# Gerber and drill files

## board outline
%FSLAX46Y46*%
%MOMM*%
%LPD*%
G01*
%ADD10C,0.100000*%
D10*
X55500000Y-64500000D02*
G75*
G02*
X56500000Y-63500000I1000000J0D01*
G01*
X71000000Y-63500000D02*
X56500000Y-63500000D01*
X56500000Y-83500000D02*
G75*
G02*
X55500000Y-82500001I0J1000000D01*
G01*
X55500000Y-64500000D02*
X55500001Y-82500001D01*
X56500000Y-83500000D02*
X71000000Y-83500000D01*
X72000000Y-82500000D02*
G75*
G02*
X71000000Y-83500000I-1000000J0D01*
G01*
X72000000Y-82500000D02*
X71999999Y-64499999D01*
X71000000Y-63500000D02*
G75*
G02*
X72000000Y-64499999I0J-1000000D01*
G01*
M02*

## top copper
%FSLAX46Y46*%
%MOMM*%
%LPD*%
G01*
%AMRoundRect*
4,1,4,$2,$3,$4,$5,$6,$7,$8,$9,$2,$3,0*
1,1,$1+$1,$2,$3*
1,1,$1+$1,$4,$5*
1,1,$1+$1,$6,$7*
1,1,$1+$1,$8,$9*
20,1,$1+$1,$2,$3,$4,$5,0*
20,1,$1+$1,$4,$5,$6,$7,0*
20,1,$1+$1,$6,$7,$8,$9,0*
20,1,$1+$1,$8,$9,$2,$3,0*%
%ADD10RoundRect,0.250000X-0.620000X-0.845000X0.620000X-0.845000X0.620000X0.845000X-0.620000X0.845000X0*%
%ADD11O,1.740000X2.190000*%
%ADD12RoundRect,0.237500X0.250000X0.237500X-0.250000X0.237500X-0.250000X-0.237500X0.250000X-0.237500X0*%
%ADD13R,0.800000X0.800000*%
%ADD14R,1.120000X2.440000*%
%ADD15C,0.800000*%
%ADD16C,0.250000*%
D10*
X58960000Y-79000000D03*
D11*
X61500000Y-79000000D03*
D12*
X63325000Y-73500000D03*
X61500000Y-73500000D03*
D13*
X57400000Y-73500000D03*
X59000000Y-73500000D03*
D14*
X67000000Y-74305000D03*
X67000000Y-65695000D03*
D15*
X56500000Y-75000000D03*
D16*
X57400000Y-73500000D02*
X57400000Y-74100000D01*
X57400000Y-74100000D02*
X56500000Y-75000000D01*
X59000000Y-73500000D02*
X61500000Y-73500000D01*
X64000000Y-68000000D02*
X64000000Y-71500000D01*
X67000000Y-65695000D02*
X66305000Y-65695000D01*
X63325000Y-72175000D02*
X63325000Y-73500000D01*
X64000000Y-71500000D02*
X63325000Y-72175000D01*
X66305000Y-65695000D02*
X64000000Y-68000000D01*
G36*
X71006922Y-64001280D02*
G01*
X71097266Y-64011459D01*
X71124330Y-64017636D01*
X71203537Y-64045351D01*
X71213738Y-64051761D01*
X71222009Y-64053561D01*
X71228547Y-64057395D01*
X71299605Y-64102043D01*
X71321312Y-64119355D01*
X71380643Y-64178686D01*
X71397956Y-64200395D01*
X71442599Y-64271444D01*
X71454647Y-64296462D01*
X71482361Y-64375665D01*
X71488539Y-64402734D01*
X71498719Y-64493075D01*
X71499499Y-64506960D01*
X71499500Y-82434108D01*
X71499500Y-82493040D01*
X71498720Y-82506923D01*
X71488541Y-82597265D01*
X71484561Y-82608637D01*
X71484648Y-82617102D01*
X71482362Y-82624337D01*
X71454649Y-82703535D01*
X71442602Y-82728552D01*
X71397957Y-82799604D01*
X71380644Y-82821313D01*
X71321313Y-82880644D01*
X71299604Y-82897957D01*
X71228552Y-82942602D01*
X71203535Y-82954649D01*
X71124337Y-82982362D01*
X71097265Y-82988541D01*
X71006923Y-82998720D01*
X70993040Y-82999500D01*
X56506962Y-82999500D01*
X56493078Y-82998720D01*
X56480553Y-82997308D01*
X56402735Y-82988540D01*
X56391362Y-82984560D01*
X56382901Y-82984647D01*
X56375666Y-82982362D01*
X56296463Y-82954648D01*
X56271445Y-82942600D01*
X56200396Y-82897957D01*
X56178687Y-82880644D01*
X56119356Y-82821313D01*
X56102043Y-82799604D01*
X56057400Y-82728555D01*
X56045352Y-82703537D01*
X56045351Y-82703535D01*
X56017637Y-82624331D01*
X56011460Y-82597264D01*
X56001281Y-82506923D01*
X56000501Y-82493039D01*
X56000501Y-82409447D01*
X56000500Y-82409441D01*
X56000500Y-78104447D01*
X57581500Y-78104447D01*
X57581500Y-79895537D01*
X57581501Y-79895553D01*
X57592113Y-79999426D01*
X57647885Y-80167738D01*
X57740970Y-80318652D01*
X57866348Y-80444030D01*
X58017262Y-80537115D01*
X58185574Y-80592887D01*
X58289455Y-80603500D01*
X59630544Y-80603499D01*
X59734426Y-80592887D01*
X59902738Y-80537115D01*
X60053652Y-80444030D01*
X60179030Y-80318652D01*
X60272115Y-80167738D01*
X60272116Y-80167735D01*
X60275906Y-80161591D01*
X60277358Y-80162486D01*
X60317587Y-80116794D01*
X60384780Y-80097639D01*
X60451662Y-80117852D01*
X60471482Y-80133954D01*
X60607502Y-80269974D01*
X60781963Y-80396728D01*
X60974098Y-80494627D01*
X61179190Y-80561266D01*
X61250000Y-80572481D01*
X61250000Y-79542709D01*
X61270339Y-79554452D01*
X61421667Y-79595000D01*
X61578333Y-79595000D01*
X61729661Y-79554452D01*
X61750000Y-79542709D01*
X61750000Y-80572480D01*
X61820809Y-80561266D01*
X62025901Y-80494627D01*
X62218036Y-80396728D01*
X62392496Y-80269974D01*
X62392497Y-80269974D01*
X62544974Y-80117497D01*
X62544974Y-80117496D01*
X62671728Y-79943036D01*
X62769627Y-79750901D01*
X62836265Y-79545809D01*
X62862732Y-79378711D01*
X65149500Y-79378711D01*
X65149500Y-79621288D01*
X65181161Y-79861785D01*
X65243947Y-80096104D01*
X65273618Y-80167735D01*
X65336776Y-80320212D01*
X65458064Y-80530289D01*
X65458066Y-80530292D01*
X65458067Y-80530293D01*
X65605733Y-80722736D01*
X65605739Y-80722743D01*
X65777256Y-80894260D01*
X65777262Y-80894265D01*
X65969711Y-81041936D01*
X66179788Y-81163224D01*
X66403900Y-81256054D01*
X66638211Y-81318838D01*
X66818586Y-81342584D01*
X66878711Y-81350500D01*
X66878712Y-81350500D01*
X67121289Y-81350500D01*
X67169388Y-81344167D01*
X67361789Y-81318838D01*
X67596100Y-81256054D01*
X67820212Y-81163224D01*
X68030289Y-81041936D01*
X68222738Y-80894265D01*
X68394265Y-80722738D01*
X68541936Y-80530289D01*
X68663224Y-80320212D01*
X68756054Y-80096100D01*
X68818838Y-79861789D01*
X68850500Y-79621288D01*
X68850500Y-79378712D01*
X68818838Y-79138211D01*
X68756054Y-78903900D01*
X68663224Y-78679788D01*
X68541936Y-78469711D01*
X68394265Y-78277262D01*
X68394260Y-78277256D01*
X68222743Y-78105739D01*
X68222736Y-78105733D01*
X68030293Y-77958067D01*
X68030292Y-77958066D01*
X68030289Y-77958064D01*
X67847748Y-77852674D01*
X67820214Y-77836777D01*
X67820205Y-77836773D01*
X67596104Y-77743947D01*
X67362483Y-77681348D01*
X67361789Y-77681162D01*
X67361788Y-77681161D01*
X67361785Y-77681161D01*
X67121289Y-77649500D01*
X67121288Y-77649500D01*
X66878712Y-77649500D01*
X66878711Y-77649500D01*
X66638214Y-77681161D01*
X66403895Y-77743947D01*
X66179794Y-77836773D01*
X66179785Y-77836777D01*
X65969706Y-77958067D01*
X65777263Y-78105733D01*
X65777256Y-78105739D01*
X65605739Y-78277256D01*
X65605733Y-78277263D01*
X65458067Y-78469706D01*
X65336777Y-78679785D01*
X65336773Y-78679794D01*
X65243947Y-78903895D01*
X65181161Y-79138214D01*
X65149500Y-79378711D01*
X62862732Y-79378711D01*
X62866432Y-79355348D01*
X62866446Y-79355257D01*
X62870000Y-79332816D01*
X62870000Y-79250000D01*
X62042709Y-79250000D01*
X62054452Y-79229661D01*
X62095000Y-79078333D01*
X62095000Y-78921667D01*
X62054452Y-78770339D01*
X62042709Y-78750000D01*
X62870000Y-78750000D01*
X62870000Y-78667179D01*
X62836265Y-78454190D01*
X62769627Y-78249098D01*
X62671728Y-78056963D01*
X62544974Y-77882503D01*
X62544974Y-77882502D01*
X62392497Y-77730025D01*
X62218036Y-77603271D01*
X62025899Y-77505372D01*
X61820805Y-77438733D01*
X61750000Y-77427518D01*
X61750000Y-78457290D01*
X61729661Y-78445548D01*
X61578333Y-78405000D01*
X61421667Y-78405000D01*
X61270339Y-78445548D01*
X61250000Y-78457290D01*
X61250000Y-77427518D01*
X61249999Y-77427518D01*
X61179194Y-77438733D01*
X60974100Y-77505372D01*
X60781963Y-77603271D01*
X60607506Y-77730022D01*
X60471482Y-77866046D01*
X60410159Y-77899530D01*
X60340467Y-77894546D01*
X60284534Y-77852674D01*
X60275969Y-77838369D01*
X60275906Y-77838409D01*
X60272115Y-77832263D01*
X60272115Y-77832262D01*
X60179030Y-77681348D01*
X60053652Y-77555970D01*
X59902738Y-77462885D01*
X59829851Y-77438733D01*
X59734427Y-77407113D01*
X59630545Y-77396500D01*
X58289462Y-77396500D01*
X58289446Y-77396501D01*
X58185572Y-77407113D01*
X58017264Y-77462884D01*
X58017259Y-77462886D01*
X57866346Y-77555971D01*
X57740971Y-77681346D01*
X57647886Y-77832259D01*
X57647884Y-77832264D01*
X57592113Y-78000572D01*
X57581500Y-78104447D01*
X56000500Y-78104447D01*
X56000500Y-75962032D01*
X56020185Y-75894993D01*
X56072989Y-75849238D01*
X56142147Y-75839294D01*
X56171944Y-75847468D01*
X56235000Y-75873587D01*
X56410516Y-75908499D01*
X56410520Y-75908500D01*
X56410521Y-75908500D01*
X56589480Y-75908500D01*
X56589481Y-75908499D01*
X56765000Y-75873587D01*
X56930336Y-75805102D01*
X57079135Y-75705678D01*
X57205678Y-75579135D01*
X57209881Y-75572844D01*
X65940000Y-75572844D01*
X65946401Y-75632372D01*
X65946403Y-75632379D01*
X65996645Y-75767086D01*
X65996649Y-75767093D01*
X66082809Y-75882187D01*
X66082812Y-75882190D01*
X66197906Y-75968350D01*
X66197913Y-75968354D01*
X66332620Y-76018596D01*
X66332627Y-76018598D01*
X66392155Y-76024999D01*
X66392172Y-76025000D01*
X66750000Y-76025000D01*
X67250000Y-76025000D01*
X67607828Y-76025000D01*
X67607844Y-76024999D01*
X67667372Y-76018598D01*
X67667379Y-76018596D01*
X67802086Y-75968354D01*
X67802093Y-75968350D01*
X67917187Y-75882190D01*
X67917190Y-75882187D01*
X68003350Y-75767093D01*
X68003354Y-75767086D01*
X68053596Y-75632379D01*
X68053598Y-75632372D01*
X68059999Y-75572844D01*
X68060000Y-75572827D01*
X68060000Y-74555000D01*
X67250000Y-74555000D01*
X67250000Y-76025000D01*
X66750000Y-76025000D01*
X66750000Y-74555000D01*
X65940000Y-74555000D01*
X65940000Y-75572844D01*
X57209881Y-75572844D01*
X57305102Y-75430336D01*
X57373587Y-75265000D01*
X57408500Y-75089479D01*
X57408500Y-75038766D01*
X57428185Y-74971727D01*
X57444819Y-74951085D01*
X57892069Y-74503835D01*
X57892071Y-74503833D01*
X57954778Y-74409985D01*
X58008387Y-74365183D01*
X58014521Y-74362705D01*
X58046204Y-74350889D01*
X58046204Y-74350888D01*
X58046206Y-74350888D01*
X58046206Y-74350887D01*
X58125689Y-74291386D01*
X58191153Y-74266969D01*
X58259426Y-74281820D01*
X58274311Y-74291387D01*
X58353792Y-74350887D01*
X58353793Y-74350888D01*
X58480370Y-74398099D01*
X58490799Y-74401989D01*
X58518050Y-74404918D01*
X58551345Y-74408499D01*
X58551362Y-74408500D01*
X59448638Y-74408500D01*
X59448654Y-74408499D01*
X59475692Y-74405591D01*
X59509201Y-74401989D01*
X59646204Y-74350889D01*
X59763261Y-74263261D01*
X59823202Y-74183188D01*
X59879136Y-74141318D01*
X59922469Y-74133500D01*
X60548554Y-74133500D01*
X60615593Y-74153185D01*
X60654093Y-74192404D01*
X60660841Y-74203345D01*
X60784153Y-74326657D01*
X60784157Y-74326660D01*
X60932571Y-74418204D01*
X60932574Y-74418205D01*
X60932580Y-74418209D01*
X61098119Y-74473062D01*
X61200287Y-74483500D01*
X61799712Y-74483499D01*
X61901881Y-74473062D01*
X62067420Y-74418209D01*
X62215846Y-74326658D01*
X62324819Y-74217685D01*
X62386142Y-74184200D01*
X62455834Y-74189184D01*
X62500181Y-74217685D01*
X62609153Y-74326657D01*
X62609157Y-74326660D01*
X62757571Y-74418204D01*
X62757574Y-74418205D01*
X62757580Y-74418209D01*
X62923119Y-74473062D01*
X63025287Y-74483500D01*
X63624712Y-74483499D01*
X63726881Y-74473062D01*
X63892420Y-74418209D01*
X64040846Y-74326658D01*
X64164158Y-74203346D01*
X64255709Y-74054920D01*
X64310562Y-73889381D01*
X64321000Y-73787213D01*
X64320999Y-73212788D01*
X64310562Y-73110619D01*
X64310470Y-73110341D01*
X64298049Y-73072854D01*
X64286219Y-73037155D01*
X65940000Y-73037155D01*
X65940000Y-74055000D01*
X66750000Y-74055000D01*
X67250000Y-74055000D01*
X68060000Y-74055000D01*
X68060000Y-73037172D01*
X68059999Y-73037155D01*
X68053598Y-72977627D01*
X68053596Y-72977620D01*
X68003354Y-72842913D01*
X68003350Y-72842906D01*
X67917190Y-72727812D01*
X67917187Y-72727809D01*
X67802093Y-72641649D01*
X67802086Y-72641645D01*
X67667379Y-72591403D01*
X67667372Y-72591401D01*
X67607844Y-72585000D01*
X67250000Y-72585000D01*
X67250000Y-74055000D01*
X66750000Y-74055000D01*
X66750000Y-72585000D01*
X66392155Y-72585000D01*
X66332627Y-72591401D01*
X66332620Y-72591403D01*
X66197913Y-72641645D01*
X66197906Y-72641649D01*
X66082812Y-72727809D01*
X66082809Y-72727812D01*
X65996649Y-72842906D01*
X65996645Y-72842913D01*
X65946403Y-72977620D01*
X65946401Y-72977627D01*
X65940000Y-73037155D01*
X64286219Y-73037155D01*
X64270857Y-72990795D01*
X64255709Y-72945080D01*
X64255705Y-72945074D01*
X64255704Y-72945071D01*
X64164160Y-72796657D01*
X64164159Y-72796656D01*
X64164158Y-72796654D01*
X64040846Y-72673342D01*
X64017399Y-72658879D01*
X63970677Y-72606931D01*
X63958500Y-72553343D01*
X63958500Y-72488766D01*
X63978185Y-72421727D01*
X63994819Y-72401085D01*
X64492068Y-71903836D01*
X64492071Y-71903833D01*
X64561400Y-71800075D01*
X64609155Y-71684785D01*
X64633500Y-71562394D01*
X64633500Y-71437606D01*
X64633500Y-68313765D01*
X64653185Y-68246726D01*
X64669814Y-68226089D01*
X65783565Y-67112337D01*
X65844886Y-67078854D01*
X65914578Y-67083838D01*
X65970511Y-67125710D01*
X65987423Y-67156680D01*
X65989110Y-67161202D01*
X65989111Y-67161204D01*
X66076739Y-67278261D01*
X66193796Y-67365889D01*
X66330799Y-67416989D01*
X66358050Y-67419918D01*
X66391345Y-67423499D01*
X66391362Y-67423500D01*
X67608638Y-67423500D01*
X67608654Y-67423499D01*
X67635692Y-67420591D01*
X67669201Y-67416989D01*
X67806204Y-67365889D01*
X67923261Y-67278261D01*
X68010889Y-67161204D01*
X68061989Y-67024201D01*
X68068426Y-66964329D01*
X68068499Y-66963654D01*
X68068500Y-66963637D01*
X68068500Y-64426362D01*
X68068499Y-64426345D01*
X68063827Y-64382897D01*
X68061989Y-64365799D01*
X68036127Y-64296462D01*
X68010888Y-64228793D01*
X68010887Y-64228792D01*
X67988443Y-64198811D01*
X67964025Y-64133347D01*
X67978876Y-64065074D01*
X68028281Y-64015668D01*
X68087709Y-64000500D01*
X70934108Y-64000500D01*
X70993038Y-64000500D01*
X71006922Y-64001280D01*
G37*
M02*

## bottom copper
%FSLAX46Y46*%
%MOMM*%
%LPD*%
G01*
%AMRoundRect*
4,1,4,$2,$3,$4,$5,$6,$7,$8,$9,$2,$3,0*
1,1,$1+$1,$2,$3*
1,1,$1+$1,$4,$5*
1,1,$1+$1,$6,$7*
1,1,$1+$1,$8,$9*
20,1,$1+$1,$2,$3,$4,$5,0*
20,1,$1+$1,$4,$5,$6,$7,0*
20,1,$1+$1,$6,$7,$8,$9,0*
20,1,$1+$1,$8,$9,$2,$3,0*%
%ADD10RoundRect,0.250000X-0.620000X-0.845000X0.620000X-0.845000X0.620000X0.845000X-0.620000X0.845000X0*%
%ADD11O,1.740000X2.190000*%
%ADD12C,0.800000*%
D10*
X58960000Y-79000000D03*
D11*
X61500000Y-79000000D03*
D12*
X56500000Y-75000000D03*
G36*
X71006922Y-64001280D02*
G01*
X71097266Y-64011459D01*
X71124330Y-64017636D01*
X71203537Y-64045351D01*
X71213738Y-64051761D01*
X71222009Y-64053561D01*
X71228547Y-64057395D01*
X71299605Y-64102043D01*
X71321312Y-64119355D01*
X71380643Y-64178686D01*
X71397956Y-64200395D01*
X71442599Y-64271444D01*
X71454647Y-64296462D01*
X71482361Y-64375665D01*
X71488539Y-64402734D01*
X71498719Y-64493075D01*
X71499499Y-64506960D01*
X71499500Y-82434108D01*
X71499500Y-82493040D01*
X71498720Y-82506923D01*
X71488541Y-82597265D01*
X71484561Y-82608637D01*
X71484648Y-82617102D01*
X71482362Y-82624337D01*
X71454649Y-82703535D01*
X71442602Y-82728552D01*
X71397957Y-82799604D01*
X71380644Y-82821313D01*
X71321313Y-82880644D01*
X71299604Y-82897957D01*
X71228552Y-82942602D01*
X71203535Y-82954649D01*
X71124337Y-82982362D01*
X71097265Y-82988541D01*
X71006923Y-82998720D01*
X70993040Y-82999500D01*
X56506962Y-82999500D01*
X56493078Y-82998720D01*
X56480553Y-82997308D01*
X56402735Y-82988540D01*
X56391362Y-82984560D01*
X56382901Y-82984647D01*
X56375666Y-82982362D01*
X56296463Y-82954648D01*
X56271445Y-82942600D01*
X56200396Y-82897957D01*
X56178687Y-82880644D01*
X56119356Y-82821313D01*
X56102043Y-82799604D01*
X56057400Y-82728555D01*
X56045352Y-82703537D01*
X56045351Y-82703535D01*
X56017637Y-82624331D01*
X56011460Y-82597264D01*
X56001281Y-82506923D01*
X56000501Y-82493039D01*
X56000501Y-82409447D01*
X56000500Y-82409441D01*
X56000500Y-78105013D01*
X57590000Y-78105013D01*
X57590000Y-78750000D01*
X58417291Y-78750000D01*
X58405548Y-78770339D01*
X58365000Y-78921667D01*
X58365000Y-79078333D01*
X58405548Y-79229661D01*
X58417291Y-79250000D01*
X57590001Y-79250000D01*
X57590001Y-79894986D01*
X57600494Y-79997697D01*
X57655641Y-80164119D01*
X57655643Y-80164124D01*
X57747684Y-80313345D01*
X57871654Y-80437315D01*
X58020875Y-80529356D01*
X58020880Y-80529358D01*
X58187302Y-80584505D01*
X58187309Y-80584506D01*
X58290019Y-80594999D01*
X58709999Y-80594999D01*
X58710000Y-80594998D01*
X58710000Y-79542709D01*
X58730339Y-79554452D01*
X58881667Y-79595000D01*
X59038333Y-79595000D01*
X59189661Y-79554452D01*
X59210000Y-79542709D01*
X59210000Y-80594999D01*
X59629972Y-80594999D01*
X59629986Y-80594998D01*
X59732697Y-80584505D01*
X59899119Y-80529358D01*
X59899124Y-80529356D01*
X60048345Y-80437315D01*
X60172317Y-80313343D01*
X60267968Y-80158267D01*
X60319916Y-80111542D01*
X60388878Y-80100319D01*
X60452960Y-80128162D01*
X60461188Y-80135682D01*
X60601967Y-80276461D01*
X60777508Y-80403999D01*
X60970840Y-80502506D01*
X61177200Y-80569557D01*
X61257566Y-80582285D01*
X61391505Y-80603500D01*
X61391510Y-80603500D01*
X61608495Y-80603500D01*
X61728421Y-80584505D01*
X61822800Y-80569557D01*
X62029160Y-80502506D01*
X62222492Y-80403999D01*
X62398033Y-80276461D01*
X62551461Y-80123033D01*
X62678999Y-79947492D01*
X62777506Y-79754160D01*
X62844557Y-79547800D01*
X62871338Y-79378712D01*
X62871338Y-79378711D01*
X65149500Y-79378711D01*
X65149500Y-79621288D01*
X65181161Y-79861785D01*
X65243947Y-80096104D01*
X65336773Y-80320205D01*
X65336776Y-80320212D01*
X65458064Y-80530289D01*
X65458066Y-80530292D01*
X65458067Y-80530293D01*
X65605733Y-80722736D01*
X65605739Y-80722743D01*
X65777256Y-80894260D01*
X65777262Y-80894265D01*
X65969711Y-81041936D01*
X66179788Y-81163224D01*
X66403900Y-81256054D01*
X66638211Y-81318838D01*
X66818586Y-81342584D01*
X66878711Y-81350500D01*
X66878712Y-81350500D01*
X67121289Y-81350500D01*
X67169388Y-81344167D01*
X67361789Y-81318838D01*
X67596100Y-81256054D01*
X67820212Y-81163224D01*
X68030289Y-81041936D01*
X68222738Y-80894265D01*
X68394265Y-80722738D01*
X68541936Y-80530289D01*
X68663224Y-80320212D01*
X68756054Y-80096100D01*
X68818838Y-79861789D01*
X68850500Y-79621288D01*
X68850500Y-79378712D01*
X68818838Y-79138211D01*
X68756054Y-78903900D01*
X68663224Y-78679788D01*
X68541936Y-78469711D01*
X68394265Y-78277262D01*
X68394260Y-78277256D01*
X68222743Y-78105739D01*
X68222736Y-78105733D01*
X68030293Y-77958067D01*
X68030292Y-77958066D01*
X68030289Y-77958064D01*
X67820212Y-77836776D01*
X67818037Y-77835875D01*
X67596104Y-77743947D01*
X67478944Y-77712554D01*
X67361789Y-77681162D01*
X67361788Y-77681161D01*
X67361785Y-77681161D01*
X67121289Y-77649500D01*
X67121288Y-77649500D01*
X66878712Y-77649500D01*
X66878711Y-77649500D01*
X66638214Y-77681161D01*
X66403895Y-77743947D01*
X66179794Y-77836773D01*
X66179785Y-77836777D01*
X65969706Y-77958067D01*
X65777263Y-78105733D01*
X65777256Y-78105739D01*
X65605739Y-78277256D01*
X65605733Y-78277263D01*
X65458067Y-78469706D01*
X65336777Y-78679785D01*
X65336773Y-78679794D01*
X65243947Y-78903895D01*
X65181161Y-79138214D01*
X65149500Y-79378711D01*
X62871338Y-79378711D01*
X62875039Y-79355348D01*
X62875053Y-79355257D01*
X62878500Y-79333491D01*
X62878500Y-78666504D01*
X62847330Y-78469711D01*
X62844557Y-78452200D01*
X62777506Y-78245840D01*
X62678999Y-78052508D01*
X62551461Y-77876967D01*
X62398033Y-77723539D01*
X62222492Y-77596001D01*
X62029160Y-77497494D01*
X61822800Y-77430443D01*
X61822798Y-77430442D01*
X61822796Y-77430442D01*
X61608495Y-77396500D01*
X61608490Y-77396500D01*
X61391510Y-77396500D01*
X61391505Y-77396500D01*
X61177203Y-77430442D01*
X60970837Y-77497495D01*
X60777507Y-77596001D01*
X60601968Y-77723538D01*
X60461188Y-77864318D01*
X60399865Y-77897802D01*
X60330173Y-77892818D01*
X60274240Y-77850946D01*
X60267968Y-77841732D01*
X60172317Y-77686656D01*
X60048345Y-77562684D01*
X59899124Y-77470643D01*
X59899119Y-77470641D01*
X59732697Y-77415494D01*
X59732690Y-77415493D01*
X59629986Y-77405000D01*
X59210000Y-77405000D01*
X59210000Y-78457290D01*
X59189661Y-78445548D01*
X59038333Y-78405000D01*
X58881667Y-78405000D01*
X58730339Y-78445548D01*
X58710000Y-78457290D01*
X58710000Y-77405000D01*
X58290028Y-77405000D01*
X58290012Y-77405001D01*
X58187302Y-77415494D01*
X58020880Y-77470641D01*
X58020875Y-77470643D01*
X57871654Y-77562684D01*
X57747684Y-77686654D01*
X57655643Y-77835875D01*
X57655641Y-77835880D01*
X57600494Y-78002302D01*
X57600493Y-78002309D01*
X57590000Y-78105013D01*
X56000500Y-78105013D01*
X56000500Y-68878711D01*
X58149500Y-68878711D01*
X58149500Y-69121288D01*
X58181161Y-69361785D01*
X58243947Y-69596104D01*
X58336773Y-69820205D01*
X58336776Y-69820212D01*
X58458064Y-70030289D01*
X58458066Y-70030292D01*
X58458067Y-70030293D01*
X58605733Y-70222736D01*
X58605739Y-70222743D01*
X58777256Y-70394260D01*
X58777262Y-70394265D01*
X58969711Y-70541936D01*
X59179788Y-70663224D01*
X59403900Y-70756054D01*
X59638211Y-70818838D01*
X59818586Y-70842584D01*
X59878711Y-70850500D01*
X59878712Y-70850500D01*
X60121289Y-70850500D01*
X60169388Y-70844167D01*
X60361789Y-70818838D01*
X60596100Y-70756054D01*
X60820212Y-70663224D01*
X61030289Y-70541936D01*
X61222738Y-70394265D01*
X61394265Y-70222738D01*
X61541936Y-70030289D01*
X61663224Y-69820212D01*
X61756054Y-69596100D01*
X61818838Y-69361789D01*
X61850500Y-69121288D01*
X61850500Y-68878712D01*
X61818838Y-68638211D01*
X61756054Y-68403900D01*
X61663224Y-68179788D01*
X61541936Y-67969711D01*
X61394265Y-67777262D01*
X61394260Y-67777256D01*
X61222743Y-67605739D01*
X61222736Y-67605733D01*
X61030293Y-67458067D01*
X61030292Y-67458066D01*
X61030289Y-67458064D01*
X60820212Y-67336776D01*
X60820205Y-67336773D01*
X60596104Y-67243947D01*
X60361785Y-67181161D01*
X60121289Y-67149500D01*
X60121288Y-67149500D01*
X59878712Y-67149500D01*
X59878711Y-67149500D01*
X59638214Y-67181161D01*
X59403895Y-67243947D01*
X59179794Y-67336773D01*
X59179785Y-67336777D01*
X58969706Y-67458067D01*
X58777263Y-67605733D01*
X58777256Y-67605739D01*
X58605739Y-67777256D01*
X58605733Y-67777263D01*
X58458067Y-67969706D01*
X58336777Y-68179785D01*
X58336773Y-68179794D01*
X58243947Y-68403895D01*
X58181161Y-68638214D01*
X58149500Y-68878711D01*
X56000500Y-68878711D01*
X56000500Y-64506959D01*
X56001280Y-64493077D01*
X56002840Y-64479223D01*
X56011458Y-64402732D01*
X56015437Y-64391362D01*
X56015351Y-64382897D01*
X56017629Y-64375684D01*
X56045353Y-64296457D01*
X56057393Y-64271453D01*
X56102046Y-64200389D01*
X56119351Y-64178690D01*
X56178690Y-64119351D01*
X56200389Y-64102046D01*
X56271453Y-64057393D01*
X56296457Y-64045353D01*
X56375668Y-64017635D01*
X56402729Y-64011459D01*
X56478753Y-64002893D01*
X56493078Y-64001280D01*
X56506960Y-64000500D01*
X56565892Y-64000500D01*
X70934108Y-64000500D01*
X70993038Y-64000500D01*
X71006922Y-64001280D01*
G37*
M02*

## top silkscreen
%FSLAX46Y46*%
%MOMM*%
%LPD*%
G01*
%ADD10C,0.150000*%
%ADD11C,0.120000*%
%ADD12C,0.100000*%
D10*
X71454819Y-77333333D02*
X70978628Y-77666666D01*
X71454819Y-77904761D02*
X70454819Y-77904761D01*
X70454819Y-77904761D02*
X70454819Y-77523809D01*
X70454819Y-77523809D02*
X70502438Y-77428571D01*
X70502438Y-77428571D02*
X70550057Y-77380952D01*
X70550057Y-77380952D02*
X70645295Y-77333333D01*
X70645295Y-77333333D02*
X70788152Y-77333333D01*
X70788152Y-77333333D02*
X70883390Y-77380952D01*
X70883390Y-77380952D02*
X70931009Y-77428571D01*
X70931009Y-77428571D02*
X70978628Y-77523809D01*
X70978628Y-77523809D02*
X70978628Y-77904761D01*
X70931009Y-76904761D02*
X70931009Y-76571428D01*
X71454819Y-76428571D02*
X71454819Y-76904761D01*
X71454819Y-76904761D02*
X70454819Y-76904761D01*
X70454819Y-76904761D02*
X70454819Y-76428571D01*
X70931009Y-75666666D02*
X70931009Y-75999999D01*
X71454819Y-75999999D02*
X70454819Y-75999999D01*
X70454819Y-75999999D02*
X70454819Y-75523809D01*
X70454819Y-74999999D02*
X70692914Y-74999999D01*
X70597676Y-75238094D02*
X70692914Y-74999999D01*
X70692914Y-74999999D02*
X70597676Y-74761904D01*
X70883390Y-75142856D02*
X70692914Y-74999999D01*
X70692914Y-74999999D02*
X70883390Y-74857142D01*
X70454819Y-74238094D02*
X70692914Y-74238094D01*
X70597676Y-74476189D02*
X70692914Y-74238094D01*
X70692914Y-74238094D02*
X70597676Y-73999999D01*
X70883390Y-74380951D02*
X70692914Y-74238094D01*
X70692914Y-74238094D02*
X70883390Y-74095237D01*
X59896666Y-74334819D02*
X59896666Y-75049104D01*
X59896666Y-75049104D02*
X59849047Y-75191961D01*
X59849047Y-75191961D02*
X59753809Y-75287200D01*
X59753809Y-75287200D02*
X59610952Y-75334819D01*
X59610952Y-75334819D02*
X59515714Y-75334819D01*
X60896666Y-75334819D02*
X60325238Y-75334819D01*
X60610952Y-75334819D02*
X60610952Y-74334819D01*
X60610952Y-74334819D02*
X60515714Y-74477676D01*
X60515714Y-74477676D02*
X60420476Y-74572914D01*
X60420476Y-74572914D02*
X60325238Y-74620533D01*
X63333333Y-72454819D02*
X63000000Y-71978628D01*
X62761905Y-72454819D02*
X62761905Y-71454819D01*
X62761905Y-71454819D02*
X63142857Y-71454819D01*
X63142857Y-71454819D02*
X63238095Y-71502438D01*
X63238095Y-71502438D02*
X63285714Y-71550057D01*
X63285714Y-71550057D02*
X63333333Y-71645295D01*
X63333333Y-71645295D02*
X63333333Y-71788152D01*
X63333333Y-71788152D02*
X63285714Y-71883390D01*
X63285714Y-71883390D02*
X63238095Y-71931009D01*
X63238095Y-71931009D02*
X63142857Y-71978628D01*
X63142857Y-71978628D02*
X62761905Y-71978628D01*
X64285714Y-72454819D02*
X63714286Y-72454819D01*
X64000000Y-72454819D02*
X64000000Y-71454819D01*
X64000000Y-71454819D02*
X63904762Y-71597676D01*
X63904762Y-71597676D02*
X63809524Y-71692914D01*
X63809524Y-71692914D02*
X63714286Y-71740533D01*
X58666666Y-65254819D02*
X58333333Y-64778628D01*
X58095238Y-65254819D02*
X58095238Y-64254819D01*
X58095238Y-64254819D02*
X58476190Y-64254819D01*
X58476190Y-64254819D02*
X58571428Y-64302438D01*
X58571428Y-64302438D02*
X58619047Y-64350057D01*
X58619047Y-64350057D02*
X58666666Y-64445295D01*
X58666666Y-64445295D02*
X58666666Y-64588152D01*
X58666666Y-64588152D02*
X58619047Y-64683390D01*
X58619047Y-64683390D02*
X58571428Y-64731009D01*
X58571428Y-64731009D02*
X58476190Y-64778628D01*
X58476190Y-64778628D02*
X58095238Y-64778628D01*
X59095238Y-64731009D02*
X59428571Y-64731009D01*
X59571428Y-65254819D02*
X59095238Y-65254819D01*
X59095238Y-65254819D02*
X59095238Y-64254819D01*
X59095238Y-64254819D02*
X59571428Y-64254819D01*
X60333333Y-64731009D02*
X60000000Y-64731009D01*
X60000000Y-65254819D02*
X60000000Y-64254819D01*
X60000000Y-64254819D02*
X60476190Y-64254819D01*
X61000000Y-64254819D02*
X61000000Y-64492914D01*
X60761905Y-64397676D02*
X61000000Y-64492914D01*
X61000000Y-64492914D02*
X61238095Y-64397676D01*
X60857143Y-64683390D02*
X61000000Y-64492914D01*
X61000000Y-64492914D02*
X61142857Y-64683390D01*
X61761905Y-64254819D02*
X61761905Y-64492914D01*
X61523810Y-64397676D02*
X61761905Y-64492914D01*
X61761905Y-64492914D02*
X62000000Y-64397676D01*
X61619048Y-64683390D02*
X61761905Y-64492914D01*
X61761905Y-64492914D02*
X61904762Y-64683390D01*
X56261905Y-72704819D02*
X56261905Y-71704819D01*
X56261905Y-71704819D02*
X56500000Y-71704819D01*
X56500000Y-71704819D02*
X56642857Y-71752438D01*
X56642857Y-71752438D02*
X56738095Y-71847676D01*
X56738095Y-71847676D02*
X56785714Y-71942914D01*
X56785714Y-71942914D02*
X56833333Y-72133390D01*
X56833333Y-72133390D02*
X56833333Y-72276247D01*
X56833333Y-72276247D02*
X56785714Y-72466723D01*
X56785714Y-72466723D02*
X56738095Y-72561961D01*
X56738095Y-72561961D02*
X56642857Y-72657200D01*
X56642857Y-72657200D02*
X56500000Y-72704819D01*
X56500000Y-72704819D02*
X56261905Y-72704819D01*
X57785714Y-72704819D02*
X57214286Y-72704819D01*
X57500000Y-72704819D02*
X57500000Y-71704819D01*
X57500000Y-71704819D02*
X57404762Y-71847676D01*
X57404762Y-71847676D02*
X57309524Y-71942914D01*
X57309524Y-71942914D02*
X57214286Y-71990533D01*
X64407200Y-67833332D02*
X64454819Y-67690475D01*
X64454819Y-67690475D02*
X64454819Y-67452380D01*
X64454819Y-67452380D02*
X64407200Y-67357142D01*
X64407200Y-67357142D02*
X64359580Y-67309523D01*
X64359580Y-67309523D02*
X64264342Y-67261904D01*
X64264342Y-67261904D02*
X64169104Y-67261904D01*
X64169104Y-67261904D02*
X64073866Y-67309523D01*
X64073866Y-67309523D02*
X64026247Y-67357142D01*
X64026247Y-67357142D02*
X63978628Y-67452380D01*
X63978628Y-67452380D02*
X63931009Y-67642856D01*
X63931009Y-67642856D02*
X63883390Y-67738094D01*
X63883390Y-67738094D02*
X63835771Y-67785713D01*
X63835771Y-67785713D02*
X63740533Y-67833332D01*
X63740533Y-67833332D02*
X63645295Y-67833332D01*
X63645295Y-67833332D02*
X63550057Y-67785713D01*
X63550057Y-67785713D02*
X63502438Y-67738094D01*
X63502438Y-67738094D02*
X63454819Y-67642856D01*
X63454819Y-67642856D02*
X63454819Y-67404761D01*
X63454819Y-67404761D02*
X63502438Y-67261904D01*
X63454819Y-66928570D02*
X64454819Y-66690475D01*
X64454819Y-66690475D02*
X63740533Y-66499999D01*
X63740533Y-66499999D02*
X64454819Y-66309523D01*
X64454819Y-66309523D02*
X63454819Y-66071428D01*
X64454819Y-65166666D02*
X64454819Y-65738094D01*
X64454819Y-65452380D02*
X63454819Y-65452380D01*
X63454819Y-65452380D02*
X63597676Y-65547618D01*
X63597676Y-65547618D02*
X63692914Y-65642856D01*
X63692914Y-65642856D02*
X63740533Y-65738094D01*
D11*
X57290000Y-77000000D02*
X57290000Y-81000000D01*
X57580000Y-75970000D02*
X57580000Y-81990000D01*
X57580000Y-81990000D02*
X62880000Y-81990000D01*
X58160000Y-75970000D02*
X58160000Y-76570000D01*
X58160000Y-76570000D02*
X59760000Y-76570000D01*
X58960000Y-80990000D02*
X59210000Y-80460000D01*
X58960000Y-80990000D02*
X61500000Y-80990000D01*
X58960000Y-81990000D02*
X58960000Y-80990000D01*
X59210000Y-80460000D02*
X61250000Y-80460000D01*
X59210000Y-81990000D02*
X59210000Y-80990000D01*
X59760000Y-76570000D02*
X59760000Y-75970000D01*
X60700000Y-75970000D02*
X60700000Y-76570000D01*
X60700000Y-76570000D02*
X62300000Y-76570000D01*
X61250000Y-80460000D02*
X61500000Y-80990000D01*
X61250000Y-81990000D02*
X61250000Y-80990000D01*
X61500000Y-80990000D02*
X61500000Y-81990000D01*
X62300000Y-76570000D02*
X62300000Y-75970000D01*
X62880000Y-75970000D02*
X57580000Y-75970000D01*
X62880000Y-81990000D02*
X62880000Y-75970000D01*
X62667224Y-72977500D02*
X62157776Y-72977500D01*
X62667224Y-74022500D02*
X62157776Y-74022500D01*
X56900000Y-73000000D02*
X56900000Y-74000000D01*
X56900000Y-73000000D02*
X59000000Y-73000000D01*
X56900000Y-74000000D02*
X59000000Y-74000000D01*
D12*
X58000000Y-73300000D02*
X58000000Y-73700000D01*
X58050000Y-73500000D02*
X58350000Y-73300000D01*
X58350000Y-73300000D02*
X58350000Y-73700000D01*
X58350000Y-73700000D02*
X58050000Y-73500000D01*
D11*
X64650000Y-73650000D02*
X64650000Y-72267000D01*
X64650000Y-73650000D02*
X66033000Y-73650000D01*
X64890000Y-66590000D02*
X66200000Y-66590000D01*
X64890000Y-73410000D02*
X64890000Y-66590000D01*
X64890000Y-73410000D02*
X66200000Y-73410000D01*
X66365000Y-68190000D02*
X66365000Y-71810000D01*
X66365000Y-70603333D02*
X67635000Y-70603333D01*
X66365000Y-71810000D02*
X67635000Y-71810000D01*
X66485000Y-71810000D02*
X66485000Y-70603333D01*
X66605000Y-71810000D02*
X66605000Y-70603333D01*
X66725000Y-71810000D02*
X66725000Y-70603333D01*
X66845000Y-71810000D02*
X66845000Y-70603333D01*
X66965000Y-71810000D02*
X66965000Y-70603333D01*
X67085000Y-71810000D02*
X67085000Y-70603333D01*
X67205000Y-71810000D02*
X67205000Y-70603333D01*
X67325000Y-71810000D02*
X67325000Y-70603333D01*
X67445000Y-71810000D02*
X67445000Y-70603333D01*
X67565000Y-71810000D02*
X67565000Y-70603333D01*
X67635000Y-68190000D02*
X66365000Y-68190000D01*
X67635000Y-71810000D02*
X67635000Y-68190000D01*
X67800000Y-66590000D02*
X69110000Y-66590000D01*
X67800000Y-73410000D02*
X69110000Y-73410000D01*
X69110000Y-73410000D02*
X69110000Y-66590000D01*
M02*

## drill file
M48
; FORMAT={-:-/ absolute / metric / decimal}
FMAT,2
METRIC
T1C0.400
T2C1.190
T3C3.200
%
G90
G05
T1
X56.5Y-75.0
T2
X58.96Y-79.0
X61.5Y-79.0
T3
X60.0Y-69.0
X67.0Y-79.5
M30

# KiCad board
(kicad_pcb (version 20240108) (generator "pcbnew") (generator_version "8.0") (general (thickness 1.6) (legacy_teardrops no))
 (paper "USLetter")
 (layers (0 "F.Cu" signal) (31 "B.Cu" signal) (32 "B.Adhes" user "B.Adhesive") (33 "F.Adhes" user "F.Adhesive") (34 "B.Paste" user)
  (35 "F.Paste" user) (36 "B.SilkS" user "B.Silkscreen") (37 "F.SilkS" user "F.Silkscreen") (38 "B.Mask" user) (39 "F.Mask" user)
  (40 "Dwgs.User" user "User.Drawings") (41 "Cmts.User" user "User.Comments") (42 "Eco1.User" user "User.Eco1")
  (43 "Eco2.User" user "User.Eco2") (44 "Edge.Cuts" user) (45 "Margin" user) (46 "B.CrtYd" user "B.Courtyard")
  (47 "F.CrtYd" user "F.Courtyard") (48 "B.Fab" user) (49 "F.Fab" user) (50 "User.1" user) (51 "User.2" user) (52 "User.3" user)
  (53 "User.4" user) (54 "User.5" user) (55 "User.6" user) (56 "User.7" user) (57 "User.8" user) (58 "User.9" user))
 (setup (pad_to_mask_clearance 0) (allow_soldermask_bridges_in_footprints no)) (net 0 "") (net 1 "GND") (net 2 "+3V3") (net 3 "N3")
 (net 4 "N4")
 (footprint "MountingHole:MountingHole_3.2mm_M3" (layer "F.Cu") (at 67 79.5)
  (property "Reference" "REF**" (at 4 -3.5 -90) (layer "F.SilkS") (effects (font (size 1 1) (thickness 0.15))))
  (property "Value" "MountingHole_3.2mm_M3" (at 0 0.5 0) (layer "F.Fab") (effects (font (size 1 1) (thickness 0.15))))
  (pad "" np_thru_hole circle (at 0 0) (size 3.2 3.2) (drill 3.2) (layers "*.Cu" "*.Mask")))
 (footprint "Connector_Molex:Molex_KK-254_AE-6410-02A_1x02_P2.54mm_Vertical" (layer "F.Cu") (at 58.96 79)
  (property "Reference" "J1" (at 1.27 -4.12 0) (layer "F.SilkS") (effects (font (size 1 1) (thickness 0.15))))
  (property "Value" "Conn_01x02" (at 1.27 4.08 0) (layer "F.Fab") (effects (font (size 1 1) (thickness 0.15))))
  (fp_line (start -1.67 -2) (end -1.67 2) (stroke (width 0.12) (type solid)) (layer "F.SilkS"))
  (fp_line (start -1.38 -3.03) (end -1.38 2.99) (stroke (width 0.12) (type solid)) (layer "F.SilkS"))
  (fp_line (start -1.38 2.99) (end 3.92 2.99) (stroke (width 0.12) (type solid)) (layer "F.SilkS"))
  (fp_line (start -0.8 -3.03) (end -0.8 -2.43) (stroke (width 0.12) (type solid)) (layer "F.SilkS"))
  (fp_line (start -0.8 -2.43) (end 0.8 -2.43) (stroke (width 0.12) (type solid)) (layer "F.SilkS"))
  (fp_line (start 0 1.99) (end 0.25 1.46) (stroke (width 0.12) (type solid)) (layer "F.SilkS"))
  (fp_line (start 0 1.99) (end 2.54 1.99) (stroke (width 0.12) (type solid)) (layer "F.SilkS"))
  (fp_line (start 0 2.99) (end 0 1.99) (stroke (width 0.12) (type solid)) (layer "F.SilkS"))
  (fp_line (start 0.25 1.46) (end 2.29 1.46) (stroke (width 0.12) (type solid)) (layer "F.SilkS"))
  (fp_line (start 0.25 2.99) (end 0.25 1.99) (stroke (width 0.12) (type solid)) (layer "F.SilkS"))
  (fp_line (start 0.8 -2.43) (end 0.8 -3.03) (stroke (width 0.12) (type solid)) (layer "F.SilkS"))
  (fp_line (start 1.74 -3.03) (end 1.74 -2.43) (stroke (width 0.12) (type solid)) (layer "F.SilkS"))
  (fp_line (start 1.74 -2.43) (end 3.34 -2.43) (stroke (width 0.12) (type solid)) (layer "F.SilkS"))
  (fp_line (start 2.29 1.46) (end 2.54 1.99) (stroke (width 0.12) (type solid)) (layer "F.SilkS"))
  (fp_line (start 2.29 2.99) (end 2.29 1.99) (stroke (width 0.12) (type solid)) (layer "F.SilkS"))
  (fp_line (start 2.54 1.99) (end 2.54 2.99) (stroke (width 0.12) (type solid)) (layer "F.SilkS"))
  (fp_line (start 3.34 -2.43) (end 3.34 -3.03) (stroke (width 0.12) (type solid)) (layer "F.SilkS"))
  (fp_line (start 3.92 -3.03) (end -1.38 -3.03) (stroke (width 0.12) (type solid)) (layer "F.SilkS"))
  (fp_line (start 3.92 2.99) (end 3.92 -3.03) (stroke (width 0.12) (type solid)) (layer "F.SilkS"))
  (pad "1" thru_hole roundrect (at 0 0) (size 1.74 2.19) (drill 1.19) (layers "*.Cu" "*.Mask") (remove_unused_layers no)
   (roundrect_rratio 0.143678) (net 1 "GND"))
  (pad "2" thru_hole oval (at 2.54 0) (size 1.74 2.19) (drill 1.19) (layers "*.Cu" "*.Mask") (remove_unused_layers no) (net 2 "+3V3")))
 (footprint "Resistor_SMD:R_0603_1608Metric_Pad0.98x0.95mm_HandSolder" (layer "F.Cu") (at 62.4125 73.5 180)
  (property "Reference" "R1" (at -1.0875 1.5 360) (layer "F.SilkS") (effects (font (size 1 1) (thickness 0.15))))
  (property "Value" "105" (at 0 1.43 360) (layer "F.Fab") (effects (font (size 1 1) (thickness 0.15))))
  (fp_line (start -0.254724 0.5225) (end 0.254724 0.5225) (stroke (width 0.12) (type solid)) (layer "F.SilkS"))
  (fp_line (start -0.254724 -0.5225) (end 0.254724 -0.5225) (stroke (width 0.12) (type solid)) (layer "F.SilkS"))
  (pad "1" smd roundrect (at -0.9125 0 180) (size 0.975 0.95) (layers "F.Cu" "F.Paste" "F.Mask") (roundrect_rratio 0.25) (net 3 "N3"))
  (pad "2" smd roundrect (at 0.9125 0 180) (size 0.975 0.95) (layers "F.Cu" "F.Paste" "F.Mask") (roundrect_rratio 0.25) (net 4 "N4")))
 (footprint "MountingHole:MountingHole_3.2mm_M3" (layer "F.Cu") (at 60 69)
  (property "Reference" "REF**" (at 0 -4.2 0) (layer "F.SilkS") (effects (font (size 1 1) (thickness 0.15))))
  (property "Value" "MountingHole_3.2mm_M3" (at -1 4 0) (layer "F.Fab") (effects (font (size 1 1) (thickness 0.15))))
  (pad "" np_thru_hole circle (at 0 0) (size 3.2 3.2) (drill 3.2) (layers "*.Cu" "*.Mask")))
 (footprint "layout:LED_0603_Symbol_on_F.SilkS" (layer "F.Cu") (at 58.2 73.5)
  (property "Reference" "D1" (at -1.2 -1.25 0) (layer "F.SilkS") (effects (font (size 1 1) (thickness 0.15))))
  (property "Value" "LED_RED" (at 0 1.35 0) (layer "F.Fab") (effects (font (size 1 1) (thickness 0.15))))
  (fp_line (start -1.3 -0.5) (end -1.3 0.5) (stroke (width 0.12) (type solid)) (layer "F.SilkS"))
  (fp_line (start -1.3 -0.5) (end 0.8 -0.5) (stroke (width 0.12) (type solid)) (layer "F.SilkS"))
  (fp_line (start -1.3 0.5) (end 0.8 0.5) (stroke (width 0.12) (type solid)) (layer "F.SilkS"))
  (fp_line (start -0.2 -0.2) (end -0.2 0.2) (stroke (width 0.1) (type solid)) (layer "F.SilkS"))
  (fp_line (start -0.15 0) (end 0.15 -0.2) (stroke (width 0.1) (type solid)) (layer "F.SilkS"))
  (fp_line (start 0.15 -0.2) (end 0.15 0.2) (stroke (width 0.1) (type solid)) (layer "F.SilkS"))
  (fp_line (start 0.15 0.2) (end -0.15 0) (stroke (width 0.1) (type solid)) (layer "F.SilkS"))
  (pad "1" smd rect (at -0.8 0 180) (size 0.8 0.8) (layers "F.Cu" "F.Paste" "F.Mask") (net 1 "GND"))
  (pad "2" smd rect (at 0.8 0 180) (size 0.8 0.8) (layers "F.Cu" "F.Paste" "F.Mask") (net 4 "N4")))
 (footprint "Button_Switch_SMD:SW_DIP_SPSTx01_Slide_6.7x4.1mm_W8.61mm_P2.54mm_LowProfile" (layer "F.Cu") (at 67 70 90)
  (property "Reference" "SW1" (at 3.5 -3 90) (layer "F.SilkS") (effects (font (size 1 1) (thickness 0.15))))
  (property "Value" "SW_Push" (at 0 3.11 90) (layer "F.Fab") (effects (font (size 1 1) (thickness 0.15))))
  (fp_line (start -3.65 -2.35) (end -2.267 -2.35) (stroke (width 0.12) (type solid)) (layer "F.SilkS"))
  (fp_line (start -3.65 -2.35) (end -3.65 -0.967) (stroke (width 0.12) (type solid)) (layer "F.SilkS"))
  (fp_line (start 3.41 -2.11) (end 3.41 -0.8) (stroke (width 0.12) (type solid)) (layer "F.SilkS"))
  (fp_line (start -3.41 -2.11) (end 3.41 -2.11) (stroke (width 0.12) (type solid)) (layer "F.SilkS"))
  (fp_line (start -3.41 -2.11) (end -3.41 -0.8) (stroke (width 0.12) (type solid)) (layer "F.SilkS"))
  (fp_line (start 1.81 -0.635) (end -1.81 -0.635) (stroke (width 0.12) (type solid)) (layer "F.SilkS"))
  (fp_line (start -0.603333 -0.635) (end -0.603333 0.635) (stroke (width 0.12) (type solid)) (layer "F.SilkS"))
  (fp_line (start -1.81 -0.635) (end -1.81 0.635) (stroke (width 0.12) (type solid)) (layer "F.SilkS"))
  (fp_line (start -1.81 -0.515) (end -0.603333 -0.515) (stroke (width 0.12) (type solid)) (layer "F.SilkS"))
  (fp_line (start -1.81 -0.395) (end -0.603333 -0.395) (stroke (width 0.12) (type solid)) (layer "F.SilkS"))
  (fp_line (start -1.81 -0.275) (end -0.603333 -0.275) (stroke (width 0.12) (type solid)) (layer "F.SilkS"))
  (fp_line (start -1.81 -0.155) (end -0.603333 -0.155) (stroke (width 0.12) (type solid)) (layer "F.SilkS"))
  (fp_line (start -1.81 -0.035) (end -0.603333 -0.035) (stroke (width 0.12) (type solid)) (layer "F.SilkS"))
  (fp_line (start -1.81 0.085) (end -0.603333 0.085) (stroke (width 0.12) (type solid)) (layer "F.SilkS"))
  (fp_line (start -1.81 0.205) (end -0.603333 0.205) (stroke (width 0.12) (type solid)) (layer "F.SilkS"))
  (fp_line (start -1.81 0.325) (end -0.603333 0.325) (stroke (width 0.12) (type solid)) (layer "F.SilkS"))
  (fp_line (start -1.81 0.445) (end -0.603333 0.445) (stroke (width 0.12) (type solid)) (layer "F.SilkS"))
  (fp_line (start -1.81 0.565) (end -0.603333 0.565) (stroke (width 0.12) (type solid)) (layer "F.SilkS"))
  (fp_line (start 1.81 0.635) (end 1.81 -0.635) (stroke (width 0.12) (type solid)) (layer "F.SilkS"))
  (fp_line (start -1.81 0.635) (end 1.81 0.635) (stroke (width 0.12) (type solid)) (layer "F.SilkS"))
  (fp_line (start 3.41 0.8) (end 3.41 2.11) (stroke (width 0.12) (type solid)) (layer "F.SilkS"))
  (fp_line (start -3.41 0.8) (end -3.41 2.11) (stroke (width 0.12) (type solid)) (layer "F.SilkS"))
  (fp_line (start -3.41 2.11) (end 3.41 2.11) (stroke (width 0.12) (type solid)) (layer "F.SilkS"))
  (pad "1" smd rect (at -4.305 0 90) (size 2.44 1.12) (layers "F.Cu" "F.Paste" "F.Mask") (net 2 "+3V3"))
  (pad "2" smd rect (at 4.305 0 90) (size 2.44 1.12) (layers "F.Cu" "F.Paste" "F.Mask") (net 3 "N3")))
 (gr_arc (start 55.5 64.5) (mid 55.792893 63.792893) (end 56.5 63.5) (stroke (width 0.1) (type default)) (layer "Edge.Cuts"))
 (gr_line (start 71 63.5) (end 56.5 63.5) (stroke (width 0.1) (type default)) (layer "Edge.Cuts"))
 (gr_arc (start 56.5 83.5) (mid 55.792894 83.207107) (end 55.500001 82.500001) (stroke (width 0.1) (type default)) (layer "Edge.Cuts"))
 (gr_line (start 55.5 64.5) (end 55.500001 82.500001) (stroke (width 0.1) (type default)) (layer "Edge.Cuts"))
 (gr_line (start 56.5 83.5) (end 71 83.5) (stroke (width 0.1) (type default)) (layer "Edge.Cuts"))
 (gr_arc (start 72 82.5) (mid 71.707107 83.207107) (end 71 83.5) (stroke (width 0.1) (type default)) (layer "Edge.Cuts"))
 (gr_line (start 72 82.5) (end 71.999999 64.499999) (stroke (width 0.1) (type default)) (layer "Edge.Cuts"))
 (gr_arc (start 71 63.5) (mid 71.707106 63.792893) (end 71.999999 64.499999) (stroke (width 0.1) (type default)) (layer "Edge.Cuts"))
 (segment (start 57.4 73.5) (end 57.4 74.1) (width 0.25) (layer "F.Cu") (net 1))
 (segment (start 57.4 74.1) (end 56.5 75) (width 0.25) (layer "F.Cu") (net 1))
 (via (at 56.5 75) (size 0.8) (drill 0.4) (layers "F.Cu" "B.Cu") (free yes) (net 1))
 (segment (start 59 73.5) (end 61.5 73.5) (width 0.25) (layer "F.Cu") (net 4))
 (segment (start 64 68) (end 64 71.5) (width 0.25) (layer "F.Cu") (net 3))
 (segment (start 67 65.695) (end 66.305 65.695) (width 0.25) (layer "F.Cu") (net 3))
 (segment (start 63.325 72.175) (end 63.325 73.5) (width 0.25) (layer "F.Cu") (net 3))
 (segment (start 64 71.5) (end 63.325 72.175) (width 0.25) (layer "F.Cu") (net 3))
 (segment (start 66.305 65.695) (end 64 68) (width 0.25) (layer "F.Cu") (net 3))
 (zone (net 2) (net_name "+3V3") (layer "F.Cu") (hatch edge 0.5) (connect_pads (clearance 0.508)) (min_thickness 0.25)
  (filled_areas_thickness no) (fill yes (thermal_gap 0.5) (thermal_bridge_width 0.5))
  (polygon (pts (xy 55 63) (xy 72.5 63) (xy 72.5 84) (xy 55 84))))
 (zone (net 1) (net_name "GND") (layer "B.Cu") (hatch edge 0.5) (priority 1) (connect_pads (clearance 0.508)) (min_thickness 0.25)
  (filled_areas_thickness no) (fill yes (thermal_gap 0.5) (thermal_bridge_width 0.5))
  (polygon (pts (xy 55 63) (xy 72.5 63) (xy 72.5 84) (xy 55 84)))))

